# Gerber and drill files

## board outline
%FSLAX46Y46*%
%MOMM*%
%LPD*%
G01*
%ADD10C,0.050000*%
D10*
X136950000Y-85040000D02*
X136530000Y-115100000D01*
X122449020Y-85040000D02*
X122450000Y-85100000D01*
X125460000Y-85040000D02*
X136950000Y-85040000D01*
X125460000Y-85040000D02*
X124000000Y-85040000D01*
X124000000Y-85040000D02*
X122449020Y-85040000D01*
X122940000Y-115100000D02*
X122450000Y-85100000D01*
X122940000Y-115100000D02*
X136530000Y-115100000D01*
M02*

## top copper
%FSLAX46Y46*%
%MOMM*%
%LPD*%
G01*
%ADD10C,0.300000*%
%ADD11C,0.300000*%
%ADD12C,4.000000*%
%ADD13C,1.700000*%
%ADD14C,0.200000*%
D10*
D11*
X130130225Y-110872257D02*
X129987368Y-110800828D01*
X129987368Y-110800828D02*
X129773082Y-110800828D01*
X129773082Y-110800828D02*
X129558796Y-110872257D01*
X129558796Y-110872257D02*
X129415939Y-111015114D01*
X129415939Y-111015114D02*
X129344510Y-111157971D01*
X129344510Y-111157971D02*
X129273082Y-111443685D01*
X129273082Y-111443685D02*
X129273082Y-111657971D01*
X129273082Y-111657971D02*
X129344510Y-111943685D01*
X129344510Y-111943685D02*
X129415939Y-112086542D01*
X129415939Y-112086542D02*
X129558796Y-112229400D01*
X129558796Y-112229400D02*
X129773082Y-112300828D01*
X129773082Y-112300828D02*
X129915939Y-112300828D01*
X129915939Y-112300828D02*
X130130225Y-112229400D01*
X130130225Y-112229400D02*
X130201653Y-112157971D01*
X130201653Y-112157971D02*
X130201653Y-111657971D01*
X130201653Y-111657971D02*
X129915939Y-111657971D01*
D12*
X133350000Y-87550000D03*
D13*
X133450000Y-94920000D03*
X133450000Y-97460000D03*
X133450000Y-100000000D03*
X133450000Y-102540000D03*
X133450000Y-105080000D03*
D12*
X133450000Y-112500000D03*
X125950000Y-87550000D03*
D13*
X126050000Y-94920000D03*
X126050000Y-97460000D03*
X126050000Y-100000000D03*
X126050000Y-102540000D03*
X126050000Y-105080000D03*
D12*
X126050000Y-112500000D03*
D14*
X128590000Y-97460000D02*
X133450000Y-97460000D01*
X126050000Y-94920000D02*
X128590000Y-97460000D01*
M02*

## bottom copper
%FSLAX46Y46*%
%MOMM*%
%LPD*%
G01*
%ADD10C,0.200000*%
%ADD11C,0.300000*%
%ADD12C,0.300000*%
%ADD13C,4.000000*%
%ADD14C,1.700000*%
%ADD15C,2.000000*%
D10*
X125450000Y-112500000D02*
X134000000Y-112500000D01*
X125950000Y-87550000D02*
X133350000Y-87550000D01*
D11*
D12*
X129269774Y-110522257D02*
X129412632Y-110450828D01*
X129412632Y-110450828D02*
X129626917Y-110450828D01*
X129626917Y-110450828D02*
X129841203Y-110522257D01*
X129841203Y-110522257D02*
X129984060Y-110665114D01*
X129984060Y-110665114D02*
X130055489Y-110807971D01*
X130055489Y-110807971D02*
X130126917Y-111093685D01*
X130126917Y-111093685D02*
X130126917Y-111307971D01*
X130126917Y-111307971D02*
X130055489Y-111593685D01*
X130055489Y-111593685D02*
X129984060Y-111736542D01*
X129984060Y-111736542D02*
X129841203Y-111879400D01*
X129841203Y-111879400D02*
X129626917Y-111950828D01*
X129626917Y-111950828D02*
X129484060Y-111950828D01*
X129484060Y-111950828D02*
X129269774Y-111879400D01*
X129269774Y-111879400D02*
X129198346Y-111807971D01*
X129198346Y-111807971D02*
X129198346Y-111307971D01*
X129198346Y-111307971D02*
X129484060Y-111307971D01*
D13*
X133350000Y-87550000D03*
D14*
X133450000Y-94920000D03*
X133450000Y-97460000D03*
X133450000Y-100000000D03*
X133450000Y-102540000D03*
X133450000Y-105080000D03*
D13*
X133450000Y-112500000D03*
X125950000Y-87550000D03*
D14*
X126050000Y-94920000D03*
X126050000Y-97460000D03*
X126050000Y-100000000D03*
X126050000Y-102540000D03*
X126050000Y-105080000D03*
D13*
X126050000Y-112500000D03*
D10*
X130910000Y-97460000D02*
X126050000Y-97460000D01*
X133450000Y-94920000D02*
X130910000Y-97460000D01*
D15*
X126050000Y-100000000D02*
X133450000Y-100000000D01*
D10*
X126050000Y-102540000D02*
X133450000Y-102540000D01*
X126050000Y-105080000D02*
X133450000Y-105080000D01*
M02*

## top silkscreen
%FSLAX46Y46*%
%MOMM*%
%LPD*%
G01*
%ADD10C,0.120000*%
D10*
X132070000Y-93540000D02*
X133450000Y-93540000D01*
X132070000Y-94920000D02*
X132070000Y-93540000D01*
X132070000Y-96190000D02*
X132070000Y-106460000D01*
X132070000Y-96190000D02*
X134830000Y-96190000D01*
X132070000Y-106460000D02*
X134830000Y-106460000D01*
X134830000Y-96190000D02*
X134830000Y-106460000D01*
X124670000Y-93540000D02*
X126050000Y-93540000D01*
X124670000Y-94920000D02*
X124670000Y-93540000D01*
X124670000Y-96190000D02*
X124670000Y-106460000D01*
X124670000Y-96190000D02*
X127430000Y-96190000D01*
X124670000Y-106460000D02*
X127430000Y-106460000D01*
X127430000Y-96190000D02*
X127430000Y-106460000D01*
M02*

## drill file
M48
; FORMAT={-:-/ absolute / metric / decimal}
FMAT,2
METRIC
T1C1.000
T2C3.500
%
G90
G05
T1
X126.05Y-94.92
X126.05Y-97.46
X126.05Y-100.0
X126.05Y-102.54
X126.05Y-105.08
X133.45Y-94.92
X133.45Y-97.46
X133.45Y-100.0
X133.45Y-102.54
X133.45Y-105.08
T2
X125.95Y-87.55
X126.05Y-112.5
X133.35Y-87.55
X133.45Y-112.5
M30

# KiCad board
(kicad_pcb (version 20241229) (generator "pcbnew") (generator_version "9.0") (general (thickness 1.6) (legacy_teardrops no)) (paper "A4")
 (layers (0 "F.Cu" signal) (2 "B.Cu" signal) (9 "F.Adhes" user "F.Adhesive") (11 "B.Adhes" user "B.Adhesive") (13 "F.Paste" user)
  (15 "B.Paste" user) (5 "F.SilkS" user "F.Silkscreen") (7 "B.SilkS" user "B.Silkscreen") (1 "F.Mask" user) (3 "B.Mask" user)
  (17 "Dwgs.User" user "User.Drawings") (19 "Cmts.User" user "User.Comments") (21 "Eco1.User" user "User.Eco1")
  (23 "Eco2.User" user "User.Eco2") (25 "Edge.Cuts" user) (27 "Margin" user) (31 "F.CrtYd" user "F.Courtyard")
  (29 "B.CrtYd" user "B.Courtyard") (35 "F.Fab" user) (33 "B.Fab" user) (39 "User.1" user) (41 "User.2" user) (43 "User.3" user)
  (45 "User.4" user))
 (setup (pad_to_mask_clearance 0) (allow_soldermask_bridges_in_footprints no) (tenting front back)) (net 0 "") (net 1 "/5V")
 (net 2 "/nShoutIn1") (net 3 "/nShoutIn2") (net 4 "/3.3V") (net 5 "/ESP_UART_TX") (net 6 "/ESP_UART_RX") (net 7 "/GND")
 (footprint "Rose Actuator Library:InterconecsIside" (layer "F.Cu") (at 133.7 100)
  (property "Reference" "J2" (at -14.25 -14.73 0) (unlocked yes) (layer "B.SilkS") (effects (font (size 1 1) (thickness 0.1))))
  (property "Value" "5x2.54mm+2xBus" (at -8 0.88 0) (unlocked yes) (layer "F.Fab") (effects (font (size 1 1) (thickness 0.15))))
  (fp_line (start -1.63 -6.46) (end -0.25 -6.46) (stroke (width 0.12) (type solid)) (layer "F.SilkS"))
  (fp_line (start -1.63 -5.08) (end -1.63 -6.46) (stroke (width 0.12) (type solid)) (layer "F.SilkS"))
  (fp_line (start -1.63 -3.81) (end -1.63 6.46) (stroke (width 0.12) (type solid)) (layer "F.SilkS"))
  (fp_line (start -1.63 -3.81) (end 1.13 -3.81) (stroke (width 0.12) (type solid)) (layer "F.SilkS"))
  (fp_line (start -1.63 6.46) (end 1.13 6.46) (stroke (width 0.12) (type solid)) (layer "F.SilkS"))
  (fp_line (start 1.13 -3.81) (end 1.13 6.46) (stroke (width 0.12) (type solid)) (layer "F.SilkS"))
  (pad "1" thru_hole circle (at -0.35 -12.45) (size 4 4) (drill 3.5) (layers "*.Cu" "*.Mask") (remove_unused_layers no) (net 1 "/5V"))
  (pad "2" thru_hole circle (at -0.25 -5.08) (size 1.7 1.7) (drill 1) (layers "*.Cu" "*.Mask") (remove_unused_layers no)
   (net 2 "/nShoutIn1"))
  (pad "3" thru_hole circle (at -0.25 -2.54) (size 1.7 1.7) (drill 1) (layers "*.Cu" "*.Mask") (remove_unused_layers no)
   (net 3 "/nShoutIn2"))
  (pad "4" thru_hole circle (at -0.25 0) (size 1.7 1.7) (drill 1) (layers "*.Cu" "*.Mask") (remove_unused_layers no) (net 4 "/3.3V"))
  (pad "5" thru_hole circle (at -0.25 2.54) (size 1.7 1.7) (drill 1) (layers "*.Cu" "*.Mask") (remove_unused_layers no)
   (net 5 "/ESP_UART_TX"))
  (pad "6" thru_hole circle (at -0.25 5.08) (size 1.7 1.7) (drill 1) (layers "*.Cu" "*.Mask") (remove_unused_layers no)
   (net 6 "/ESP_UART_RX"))
  (pad "7" thru_hole circle (at -0.25 12.5) (size 4 4) (drill 3.5) (layers "*.Cu" "*.Mask") (remove_unused_layers no) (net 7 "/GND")))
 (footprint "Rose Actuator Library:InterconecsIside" (layer "F.Cu") (at 126.3 100)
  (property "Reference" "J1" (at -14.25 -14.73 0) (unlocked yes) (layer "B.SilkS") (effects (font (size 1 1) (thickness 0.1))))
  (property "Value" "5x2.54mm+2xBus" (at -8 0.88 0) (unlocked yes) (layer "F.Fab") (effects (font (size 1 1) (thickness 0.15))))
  (fp_line (start -1.63 -6.46) (end -0.25 -6.46) (stroke (width 0.12) (type solid)) (layer "F.SilkS"))
  (fp_line (start -1.63 -5.08) (end -1.63 -6.46) (stroke (width 0.12) (type solid)) (layer "F.SilkS"))
  (fp_line (start -1.63 -3.81) (end -1.63 6.46) (stroke (width 0.12) (type solid)) (layer "F.SilkS"))
  (fp_line (start -1.63 -3.81) (end 1.13 -3.81) (stroke (width 0.12) (type solid)) (layer "F.SilkS"))
  (fp_line (start -1.63 6.46) (end 1.13 6.46) (stroke (width 0.12) (type solid)) (layer "F.SilkS"))
  (fp_line (start 1.13 -3.81) (end 1.13 6.46) (stroke (width 0.12) (type solid)) (layer "F.SilkS"))
  (pad "1" thru_hole circle (at -0.35 -12.45) (size 4 4) (drill 3.5) (layers "*.Cu" "*.Mask") (remove_unused_layers no) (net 1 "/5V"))
  (pad "2" thru_hole circle (at -0.25 -5.08) (size 1.7 1.7) (drill 1) (layers "*.Cu" "*.Mask") (remove_unused_layers no)
   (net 3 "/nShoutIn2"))
  (pad "3" thru_hole circle (at -0.25 -2.54) (size 1.7 1.7) (drill 1) (layers "*.Cu" "*.Mask") (remove_unused_layers no)
   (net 2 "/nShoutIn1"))
  (pad "4" thru_hole circle (at -0.25 0) (size 1.7 1.7) (drill 1) (layers "*.Cu" "*.Mask") (remove_unused_layers no) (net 4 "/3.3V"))
  (pad "5" thru_hole circle (at -0.25 2.54) (size 1.7 1.7) (drill 1) (layers "*.Cu" "*.Mask") (remove_unused_layers no)
   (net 5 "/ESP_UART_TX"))
  (pad "6" thru_hole circle (at -0.25 5.08) (size 1.7 1.7) (drill 1) (layers "*.Cu" "*.Mask") (remove_unused_layers no)
   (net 6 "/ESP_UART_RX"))
  (pad "7" thru_hole circle (at -0.25 12.5) (size 4 4) (drill 3.5) (layers "*.Cu" "*.Mask") (remove_unused_layers no) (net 7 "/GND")))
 (gr_line (start 125.45 112.5) (end 134 112.5) (stroke (width 0.2) (type default)) (layer "B.Cu") (net 7))
 (gr_line (start 125.95 87.55) (end 133.35 87.55) (stroke (width 0.2) (type default)) (layer "B.Cu") (net 1))
 (gr_line (start 136.95 85.04) (end 136.53 115.1) (stroke (width 0.05) (type default)) (layer "Edge.Cuts"))
 (gr_line (start 122.44902 85.04) (end 122.45 85.1) (stroke (width 0.05) (type default)) (layer "Edge.Cuts"))
 (gr_line (start 125.46 85.04) (end 136.95 85.04) (stroke (width 0.05) (type default)) (layer "Edge.Cuts"))
 (gr_line (start 125.46 85.04) (end 124 85.04) (stroke (width 0.05) (type default)) (layer "Edge.Cuts"))
 (gr_line (start 124 85.04) (end 122.44902 85.04) (stroke (width 0.05) (type default)) (layer "Edge.Cuts"))
 (gr_line (start 122.94 115.1) (end 122.45 85.1) (stroke (width 0.05) (type default)) (layer "Edge.Cuts"))
 (gr_line (start 122.94 115.1) (end 136.53 115.1) (stroke (width 0.05) (type default)) (layer "Edge.Cuts"))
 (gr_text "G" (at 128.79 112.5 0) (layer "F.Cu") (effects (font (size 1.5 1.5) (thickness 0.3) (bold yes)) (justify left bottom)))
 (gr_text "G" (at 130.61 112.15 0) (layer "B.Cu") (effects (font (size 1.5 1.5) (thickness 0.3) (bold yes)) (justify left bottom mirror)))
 (segment (start 130.91 97.46) (end 126.05 97.46) (width 0.2) (layer "B.Cu") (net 2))
 (segment (start 133.45 94.92) (end 130.91 97.46) (width 0.2) (layer "B.Cu") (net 2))
 (segment (start 126.05 100) (end 133.45 100) (width 2) (layer "B.Cu") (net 4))
 (segment (start 126.05 102.54) (end 133.45 102.54) (width 0.2) (layer "B.Cu") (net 5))
 (segment (start 126.05 105.08) (end 133.45 105.08) (width 0.2) (layer "B.Cu") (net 6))
 (segment (start 128.59 97.46) (end 133.45 97.46) (width 0.2) (layer "F.Cu") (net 3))
 (segment (start 126.05 94.92) (end 128.59 97.46) (width 0.2) (layer "F.Cu") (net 3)))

